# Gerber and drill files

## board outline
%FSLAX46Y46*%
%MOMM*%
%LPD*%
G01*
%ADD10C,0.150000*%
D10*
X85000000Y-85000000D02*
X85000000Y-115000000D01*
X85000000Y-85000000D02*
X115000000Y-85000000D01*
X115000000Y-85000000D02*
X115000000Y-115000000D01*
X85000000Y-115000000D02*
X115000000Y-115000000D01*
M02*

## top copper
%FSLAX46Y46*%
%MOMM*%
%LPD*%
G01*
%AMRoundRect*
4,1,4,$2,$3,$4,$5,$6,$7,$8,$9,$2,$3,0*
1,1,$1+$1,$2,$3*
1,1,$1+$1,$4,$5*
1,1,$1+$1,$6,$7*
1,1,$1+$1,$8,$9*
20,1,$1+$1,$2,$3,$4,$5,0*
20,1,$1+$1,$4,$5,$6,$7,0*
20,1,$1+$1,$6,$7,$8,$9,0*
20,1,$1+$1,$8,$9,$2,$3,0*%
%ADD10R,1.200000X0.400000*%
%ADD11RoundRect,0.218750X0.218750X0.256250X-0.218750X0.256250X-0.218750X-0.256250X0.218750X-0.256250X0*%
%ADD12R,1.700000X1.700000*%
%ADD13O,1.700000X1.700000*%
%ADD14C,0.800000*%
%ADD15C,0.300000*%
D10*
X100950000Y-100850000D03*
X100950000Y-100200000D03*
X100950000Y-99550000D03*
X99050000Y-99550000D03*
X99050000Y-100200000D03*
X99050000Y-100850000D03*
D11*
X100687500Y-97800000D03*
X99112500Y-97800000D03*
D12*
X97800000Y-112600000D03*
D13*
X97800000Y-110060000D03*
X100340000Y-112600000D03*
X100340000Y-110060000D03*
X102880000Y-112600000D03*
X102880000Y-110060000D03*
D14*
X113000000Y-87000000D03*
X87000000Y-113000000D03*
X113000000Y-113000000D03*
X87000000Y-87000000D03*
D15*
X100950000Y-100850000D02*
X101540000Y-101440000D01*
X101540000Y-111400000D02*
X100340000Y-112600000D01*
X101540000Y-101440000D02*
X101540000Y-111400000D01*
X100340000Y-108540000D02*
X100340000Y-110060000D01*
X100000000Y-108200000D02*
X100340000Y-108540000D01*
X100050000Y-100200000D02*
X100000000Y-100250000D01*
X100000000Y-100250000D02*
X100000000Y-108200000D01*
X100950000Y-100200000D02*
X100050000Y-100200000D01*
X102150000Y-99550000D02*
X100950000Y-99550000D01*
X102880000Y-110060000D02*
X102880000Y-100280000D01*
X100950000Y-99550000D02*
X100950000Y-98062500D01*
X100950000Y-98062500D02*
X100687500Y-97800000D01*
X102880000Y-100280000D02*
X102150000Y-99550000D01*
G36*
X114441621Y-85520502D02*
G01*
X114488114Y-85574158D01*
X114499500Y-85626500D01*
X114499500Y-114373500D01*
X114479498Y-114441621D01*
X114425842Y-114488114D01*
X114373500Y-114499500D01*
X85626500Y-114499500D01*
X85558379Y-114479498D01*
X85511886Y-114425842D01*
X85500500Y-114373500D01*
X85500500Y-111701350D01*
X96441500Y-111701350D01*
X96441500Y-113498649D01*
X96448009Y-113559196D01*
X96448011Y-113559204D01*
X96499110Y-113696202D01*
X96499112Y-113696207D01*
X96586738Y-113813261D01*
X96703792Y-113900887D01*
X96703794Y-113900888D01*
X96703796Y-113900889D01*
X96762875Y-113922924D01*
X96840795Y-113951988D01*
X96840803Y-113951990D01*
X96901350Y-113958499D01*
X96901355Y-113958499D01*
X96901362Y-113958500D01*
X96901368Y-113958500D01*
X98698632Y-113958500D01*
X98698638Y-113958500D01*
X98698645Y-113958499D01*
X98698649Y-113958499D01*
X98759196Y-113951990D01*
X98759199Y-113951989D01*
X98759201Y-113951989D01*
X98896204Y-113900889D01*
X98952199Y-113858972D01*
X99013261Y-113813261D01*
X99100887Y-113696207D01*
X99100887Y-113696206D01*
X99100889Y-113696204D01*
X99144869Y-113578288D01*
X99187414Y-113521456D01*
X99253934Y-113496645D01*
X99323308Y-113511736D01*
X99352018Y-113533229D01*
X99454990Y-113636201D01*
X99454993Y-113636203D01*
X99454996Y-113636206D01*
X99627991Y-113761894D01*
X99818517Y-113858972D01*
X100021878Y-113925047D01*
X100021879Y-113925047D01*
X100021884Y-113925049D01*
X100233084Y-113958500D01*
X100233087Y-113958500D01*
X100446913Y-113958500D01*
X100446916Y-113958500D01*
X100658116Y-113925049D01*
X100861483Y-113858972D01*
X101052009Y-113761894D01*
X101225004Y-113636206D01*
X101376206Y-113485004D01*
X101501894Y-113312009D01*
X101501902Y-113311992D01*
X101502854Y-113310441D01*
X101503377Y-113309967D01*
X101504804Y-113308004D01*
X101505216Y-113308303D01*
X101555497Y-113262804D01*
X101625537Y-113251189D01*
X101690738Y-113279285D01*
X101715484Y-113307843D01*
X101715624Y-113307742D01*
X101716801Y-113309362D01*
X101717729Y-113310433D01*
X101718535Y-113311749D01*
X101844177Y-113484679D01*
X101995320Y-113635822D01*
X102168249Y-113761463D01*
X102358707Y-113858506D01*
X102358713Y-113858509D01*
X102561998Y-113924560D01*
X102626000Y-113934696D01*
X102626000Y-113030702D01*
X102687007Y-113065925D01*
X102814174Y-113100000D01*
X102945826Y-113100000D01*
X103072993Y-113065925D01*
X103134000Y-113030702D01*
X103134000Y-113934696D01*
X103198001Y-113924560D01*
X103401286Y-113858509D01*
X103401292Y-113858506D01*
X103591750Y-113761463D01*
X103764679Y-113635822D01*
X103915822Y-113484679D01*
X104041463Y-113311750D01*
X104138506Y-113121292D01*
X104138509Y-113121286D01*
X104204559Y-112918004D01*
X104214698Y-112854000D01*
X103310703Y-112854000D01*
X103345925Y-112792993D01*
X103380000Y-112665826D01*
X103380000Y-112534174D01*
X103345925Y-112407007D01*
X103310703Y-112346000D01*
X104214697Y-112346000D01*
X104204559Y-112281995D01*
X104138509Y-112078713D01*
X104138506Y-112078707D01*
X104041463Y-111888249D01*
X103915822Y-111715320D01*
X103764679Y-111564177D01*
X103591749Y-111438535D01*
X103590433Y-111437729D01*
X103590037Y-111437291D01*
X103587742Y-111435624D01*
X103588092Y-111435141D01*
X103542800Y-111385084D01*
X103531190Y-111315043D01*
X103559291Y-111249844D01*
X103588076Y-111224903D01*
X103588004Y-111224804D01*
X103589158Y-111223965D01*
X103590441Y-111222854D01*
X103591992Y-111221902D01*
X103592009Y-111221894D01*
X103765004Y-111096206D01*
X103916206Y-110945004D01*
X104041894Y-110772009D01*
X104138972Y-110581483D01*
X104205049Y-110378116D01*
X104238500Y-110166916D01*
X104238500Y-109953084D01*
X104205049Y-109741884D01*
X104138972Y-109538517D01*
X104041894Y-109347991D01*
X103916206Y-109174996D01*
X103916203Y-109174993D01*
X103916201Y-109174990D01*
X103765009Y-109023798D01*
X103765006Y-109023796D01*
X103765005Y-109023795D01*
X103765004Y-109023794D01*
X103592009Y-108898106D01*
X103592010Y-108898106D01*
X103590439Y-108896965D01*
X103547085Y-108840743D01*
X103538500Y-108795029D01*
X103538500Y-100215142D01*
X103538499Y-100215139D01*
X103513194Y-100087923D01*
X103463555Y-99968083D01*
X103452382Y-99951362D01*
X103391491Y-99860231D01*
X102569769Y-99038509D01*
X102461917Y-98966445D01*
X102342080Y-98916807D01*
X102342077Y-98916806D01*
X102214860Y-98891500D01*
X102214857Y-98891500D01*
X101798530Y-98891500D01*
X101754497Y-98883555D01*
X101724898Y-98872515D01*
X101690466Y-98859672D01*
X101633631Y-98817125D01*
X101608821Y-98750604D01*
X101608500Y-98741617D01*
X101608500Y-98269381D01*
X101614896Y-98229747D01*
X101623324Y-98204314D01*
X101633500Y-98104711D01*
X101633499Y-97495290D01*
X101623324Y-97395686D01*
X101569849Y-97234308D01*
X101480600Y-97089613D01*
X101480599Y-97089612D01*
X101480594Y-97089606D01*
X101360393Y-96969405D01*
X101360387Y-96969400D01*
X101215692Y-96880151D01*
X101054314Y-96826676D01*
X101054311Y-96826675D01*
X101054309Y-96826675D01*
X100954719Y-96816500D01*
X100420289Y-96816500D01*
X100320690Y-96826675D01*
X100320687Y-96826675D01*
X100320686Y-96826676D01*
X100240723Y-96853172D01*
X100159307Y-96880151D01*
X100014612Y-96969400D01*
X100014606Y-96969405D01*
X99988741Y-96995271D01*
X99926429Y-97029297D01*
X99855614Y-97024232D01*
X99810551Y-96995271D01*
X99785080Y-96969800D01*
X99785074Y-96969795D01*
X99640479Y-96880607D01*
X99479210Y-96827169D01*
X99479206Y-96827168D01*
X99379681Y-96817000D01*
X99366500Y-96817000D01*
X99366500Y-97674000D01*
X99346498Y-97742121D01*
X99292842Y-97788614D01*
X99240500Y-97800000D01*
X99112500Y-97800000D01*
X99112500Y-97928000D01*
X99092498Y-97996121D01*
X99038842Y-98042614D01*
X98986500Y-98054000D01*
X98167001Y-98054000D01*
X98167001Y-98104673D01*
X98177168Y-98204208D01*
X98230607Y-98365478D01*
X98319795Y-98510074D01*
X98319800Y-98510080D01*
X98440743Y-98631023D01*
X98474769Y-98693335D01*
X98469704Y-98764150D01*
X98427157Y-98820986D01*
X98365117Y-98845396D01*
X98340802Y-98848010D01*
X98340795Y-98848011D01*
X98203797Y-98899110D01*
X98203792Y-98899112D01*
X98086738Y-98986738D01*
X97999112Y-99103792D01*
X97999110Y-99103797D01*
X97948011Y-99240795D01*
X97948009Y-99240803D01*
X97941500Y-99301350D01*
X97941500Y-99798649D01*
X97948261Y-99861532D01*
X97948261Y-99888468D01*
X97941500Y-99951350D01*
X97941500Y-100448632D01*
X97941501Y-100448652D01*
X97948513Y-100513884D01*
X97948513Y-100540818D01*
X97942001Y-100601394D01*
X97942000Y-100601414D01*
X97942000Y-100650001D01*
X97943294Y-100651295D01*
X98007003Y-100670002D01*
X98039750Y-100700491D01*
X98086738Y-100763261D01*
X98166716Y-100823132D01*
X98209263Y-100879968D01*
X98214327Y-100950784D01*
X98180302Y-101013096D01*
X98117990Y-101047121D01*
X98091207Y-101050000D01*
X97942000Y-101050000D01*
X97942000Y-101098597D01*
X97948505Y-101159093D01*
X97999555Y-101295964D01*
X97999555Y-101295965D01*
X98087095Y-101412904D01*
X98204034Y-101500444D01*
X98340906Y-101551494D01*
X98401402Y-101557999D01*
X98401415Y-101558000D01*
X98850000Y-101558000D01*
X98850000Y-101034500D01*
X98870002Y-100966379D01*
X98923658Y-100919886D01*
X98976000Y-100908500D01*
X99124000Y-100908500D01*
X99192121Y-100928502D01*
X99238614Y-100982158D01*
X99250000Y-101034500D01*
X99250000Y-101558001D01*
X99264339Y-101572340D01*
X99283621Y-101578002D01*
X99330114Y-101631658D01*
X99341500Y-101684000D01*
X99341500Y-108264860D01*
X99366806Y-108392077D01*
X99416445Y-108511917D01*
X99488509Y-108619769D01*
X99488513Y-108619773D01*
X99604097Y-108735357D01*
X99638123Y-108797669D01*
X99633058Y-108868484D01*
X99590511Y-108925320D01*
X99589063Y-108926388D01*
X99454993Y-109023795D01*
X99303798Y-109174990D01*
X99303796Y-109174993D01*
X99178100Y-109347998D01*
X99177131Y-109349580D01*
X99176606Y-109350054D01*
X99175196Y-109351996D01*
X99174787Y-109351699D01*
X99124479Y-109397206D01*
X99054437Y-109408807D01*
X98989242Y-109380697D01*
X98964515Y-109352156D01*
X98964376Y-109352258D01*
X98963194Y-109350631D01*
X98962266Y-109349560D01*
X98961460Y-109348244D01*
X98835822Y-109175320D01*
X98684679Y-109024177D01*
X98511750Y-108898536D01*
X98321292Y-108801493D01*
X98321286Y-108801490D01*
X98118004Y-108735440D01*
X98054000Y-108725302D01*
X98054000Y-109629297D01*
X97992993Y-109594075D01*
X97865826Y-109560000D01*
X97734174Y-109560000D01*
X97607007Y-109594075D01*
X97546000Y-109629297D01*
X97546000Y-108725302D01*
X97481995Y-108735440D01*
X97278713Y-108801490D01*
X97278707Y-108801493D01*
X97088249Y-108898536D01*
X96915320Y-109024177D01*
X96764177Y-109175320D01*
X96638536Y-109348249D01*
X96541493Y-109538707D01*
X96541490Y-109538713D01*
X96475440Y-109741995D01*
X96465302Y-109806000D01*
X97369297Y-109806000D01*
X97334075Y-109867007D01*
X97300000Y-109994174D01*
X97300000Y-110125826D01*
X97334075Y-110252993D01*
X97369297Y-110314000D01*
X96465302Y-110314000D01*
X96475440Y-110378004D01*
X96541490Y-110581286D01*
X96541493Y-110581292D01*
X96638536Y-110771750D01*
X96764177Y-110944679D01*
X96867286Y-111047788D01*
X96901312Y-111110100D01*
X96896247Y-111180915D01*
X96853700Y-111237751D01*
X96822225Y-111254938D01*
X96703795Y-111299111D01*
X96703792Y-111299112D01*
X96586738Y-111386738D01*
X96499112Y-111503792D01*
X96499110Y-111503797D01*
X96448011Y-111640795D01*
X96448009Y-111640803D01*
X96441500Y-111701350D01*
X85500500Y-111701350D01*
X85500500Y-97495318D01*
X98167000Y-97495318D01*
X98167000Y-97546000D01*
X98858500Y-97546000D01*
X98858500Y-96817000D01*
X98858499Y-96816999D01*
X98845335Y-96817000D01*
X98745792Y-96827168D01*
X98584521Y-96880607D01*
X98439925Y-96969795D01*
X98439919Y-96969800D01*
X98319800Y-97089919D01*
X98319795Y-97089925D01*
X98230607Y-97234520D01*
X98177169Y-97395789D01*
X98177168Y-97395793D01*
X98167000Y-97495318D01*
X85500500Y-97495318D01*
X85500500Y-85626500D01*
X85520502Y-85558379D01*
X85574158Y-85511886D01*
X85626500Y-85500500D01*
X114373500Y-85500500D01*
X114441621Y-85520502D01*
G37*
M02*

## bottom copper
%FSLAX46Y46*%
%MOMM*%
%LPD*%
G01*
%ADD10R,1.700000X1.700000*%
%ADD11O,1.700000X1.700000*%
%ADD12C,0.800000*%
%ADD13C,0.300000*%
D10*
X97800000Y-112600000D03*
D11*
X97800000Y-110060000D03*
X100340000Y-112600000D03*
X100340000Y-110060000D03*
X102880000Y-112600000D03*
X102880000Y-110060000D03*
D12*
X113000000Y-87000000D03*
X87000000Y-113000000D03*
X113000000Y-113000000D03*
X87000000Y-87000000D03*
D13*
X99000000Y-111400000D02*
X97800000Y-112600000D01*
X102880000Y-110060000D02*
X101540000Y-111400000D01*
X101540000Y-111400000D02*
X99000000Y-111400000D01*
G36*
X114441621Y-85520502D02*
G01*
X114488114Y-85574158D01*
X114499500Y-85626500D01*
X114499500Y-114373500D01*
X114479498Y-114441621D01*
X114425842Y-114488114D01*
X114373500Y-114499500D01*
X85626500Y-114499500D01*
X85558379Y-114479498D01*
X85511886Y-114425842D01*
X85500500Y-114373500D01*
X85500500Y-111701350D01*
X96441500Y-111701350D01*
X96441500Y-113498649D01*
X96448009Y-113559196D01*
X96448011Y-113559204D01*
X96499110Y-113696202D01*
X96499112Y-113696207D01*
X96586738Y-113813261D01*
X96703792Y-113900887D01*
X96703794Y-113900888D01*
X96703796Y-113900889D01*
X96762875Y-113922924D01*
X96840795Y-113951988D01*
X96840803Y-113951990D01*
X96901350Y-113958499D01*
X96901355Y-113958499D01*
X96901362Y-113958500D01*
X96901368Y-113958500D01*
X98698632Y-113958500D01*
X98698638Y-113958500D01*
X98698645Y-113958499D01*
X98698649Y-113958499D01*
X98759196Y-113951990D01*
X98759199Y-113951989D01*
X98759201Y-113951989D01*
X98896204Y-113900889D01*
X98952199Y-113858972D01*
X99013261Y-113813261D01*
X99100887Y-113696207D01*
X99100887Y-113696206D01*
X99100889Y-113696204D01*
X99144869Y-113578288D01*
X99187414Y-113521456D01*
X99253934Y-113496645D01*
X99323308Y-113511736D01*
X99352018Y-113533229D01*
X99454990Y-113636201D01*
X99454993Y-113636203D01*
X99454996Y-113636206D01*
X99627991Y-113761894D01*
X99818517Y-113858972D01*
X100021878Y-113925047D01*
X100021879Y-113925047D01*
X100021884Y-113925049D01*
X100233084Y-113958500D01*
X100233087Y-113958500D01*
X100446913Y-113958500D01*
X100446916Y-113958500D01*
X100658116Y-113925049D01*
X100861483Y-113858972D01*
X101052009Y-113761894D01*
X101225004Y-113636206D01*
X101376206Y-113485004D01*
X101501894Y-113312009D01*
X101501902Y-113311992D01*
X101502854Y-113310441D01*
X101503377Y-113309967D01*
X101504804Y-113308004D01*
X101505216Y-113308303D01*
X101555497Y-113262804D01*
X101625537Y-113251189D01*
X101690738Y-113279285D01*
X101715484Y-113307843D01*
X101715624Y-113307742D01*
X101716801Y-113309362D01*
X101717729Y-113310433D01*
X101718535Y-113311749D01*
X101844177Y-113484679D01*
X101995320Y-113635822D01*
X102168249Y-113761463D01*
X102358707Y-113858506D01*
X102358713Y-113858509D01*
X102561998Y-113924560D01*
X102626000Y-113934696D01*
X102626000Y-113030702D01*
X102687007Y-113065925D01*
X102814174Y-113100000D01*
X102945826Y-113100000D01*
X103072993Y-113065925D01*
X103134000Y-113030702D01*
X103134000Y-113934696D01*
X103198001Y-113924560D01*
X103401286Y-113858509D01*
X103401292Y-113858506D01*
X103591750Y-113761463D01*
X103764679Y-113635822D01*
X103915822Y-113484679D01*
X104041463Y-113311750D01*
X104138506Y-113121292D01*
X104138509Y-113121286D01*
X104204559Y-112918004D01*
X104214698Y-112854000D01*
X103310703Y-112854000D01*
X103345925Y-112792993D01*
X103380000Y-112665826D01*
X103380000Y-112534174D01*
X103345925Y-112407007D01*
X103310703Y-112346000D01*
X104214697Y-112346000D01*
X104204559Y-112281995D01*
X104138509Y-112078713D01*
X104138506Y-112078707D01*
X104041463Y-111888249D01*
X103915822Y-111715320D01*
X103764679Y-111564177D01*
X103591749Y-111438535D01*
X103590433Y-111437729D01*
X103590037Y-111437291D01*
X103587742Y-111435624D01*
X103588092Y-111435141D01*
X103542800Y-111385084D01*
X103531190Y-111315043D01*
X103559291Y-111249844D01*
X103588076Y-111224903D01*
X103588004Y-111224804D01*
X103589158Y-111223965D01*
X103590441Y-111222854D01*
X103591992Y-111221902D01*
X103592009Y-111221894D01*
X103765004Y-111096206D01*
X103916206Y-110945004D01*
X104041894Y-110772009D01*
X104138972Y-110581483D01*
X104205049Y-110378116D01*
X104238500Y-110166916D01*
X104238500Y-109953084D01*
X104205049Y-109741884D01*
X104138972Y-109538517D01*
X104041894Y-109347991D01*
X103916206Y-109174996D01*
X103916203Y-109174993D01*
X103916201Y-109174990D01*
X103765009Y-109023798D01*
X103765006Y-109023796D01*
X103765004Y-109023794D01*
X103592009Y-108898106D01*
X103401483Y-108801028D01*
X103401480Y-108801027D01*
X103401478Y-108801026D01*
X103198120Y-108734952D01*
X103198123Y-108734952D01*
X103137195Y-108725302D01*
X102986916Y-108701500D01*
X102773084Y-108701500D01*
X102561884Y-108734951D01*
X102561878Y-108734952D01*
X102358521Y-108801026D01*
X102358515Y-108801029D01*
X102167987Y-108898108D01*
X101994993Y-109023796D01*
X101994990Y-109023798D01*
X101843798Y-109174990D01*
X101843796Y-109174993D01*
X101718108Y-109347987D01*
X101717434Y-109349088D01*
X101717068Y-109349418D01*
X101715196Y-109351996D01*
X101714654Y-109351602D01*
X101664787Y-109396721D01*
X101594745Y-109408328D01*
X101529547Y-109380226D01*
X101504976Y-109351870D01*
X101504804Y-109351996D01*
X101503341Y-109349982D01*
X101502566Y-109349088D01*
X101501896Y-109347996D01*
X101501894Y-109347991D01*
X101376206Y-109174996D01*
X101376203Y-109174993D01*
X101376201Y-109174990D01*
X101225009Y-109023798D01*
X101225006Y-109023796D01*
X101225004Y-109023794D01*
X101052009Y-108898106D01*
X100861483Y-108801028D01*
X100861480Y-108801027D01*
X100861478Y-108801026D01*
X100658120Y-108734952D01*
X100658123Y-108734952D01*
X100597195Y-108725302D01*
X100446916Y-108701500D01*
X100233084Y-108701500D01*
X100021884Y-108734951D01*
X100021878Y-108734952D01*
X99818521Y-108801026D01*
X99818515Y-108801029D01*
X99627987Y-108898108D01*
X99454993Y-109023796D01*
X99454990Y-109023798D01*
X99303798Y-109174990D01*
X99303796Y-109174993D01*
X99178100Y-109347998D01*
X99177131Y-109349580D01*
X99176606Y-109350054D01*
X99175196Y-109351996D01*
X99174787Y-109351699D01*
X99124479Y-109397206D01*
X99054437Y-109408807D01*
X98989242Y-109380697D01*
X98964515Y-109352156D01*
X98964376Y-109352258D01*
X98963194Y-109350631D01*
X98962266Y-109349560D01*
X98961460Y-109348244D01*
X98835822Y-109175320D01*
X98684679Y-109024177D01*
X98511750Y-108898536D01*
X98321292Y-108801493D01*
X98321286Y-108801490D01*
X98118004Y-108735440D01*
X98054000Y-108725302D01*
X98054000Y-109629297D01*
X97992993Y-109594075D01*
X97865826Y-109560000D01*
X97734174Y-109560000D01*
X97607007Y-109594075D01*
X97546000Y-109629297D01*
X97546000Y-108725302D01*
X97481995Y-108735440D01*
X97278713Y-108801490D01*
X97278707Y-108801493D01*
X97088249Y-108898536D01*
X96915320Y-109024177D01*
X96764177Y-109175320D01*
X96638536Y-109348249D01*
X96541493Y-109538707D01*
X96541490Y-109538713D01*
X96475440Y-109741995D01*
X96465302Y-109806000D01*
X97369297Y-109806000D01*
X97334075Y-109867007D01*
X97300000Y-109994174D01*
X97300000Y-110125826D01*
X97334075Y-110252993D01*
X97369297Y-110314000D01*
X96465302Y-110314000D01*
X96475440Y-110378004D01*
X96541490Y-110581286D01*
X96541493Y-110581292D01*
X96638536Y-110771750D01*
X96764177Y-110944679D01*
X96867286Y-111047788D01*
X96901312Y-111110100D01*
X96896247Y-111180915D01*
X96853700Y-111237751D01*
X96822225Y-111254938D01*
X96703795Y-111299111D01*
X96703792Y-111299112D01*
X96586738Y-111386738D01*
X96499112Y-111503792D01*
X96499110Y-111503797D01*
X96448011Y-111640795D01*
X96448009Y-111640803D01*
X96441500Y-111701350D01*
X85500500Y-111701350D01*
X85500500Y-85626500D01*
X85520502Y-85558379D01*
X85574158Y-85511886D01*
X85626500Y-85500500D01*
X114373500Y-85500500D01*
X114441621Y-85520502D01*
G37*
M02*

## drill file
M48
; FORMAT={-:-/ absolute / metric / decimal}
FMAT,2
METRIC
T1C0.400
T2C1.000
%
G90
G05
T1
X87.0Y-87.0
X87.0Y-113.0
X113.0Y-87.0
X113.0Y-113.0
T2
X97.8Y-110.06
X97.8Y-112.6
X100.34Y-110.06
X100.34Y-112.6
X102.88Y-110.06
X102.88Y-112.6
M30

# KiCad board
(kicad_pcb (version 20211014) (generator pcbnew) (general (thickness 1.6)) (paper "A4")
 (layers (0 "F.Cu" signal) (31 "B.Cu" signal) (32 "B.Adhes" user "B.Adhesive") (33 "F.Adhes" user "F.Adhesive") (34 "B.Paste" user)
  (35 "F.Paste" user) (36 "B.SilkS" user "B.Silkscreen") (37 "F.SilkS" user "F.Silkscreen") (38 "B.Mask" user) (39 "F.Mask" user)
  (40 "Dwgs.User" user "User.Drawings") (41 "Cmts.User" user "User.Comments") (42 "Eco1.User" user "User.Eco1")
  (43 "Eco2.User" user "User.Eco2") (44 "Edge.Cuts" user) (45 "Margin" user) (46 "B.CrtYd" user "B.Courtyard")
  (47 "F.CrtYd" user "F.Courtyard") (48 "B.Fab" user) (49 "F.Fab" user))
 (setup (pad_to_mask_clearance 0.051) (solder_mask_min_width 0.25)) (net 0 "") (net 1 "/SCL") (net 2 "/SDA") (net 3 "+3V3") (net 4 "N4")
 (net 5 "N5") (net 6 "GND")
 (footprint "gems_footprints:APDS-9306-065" (layer "F.Cu") (at 100 100.2 -90)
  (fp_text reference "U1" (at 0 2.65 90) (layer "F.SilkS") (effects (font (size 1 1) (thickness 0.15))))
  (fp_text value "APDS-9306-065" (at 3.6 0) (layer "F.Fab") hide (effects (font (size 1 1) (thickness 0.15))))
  (pad "1" smd rect (at 0.65 -0.95 270) (size 0.4 1.2) (layers "F.Cu" "F.Paste" "F.Mask") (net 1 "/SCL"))
  (pad "2" smd rect (at 0 -0.95 270) (size 0.4 1.2) (layers "F.Cu" "F.Paste" "F.Mask") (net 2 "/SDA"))
  (pad "3" smd rect (at -0.65 -0.95 270) (size 0.4 1.2) (layers "F.Cu" "F.Paste" "F.Mask") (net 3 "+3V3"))
  (pad "4" smd rect (at -0.65 0.95 270) (size 0.4 1.2) (layers "F.Cu" "F.Paste" "F.Mask") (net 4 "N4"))
  (pad "5" smd rect (at 0 0.95 270) (size 0.4 1.2) (layers "F.Cu" "F.Paste" "F.Mask") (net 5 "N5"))
  (pad "6" smd rect (at 0.65 0.95 270) (size 0.4 1.2) (layers "F.Cu" "F.Paste" "F.Mask") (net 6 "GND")))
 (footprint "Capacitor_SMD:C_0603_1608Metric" (layer "F.Cu") (at 99.9 97.8 180)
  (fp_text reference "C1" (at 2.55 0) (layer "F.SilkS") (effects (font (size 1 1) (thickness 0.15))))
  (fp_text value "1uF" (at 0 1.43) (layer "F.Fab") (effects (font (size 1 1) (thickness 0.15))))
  (pad "1" smd roundrect locked (at -0.7875 0 180) (size 0.875 0.95) (layers "F.Cu" "F.Paste" "F.Mask") (roundrect_rratio 0.25)
   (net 3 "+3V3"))
  (pad "2" smd roundrect locked (at 0.7875 0 180) (size 0.875 0.95) (layers "F.Cu" "F.Paste" "F.Mask") (roundrect_rratio 0.25) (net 6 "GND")))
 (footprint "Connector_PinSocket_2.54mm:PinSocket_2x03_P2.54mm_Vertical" (layer "B.Cu") (at 97.8 112.6 -90)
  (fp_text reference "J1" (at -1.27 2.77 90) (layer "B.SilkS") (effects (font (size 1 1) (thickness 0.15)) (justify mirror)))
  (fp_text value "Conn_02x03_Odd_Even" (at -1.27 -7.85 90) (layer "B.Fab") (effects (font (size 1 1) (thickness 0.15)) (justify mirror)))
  (pad "1" thru_hole rect (at 0 0 270) (size 1.7 1.7) (drill 1) (layers *.Cu *.Mask) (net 3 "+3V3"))
  (pad "2" thru_hole oval (at -2.54 0 270) (size 1.7 1.7) (drill 1) (layers *.Cu *.Mask) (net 6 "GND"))
  (pad "3" thru_hole oval (at 0 -2.54 270) (size 1.7 1.7) (drill 1) (layers *.Cu *.Mask) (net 1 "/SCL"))
  (pad "4" thru_hole oval (at -2.54 -2.54 270) (size 1.7 1.7) (drill 1) (layers *.Cu *.Mask) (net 2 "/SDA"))
  (pad "5" thru_hole oval (at 0 -5.08 270) (size 1.7 1.7) (drill 1) (layers *.Cu *.Mask) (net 6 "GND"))
  (pad "6" thru_hole oval (at -2.54 -5.08 270) (size 1.7 1.7) (drill 1) (layers *.Cu *.Mask) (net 3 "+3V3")))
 (gr_line (start 85 85) (end 85 115) (layer "Edge.Cuts") (width 0.15))
 (gr_line (start 85 85) (end 115 85) (layer "Edge.Cuts") (width 0.15))
 (gr_line (start 115 85) (end 115 115) (layer "Edge.Cuts") (width 0.15))
 (gr_line (start 85 115) (end 115 115) (layer "Edge.Cuts") (width 0.15))
 (segment (start 100.95 100.85) (end 101.54 101.44) (width 0.3) (layer "F.Cu") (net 1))
 (segment (start 101.54 111.4) (end 100.34 112.6) (width 0.3) (layer "F.Cu") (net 1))
 (segment (start 101.54 101.44) (end 101.54 111.4) (width 0.3) (layer "F.Cu") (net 1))
 (segment (start 100.34 108.54) (end 100.34 110.06) (width 0.3) (layer "F.Cu") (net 2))
 (segment (start 100 108.2) (end 100.34 108.54) (width 0.3) (layer "F.Cu") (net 2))
 (segment (start 100.05 100.2) (end 100 100.25) (width 0.3) (layer "F.Cu") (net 2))
 (segment (start 100 100.25) (end 100 108.2) (width 0.3) (layer "F.Cu") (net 2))
 (segment (start 100.95 100.2) (end 100.05 100.2) (width 0.3) (layer "F.Cu") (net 2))
 (segment (start 102.15 99.55) (end 100.95 99.55) (width 0.3) (layer "F.Cu") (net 3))
 (segment (start 102.88 110.06) (end 102.88 100.28) (width 0.3) (layer "F.Cu") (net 3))
 (segment (start 100.95 99.55) (end 100.95 98.0625) (width 0.3) (layer "F.Cu") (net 3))
 (segment (start 100.95 98.0625) (end 100.6875 97.8) (width 0.3) (layer "F.Cu") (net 3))
 (segment (start 102.88 100.28) (end 102.15 99.55) (width 0.3) (layer "F.Cu") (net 3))
 (segment (start 99 111.4) (end 97.8 112.6) (width 0.3) (layer "B.Cu") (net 3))
 (segment (start 102.88 110.06) (end 101.54 111.4) (width 0.3) (layer "B.Cu") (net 3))
 (segment (start 101.54 111.4) (end 99 111.4) (width 0.3) (layer "B.Cu") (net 3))
 (via (at 113 87) (size 0.8) (drill 0.4) (layers "F.Cu" "B.Cu") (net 6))
 (via (at 87 113) (size 0.8) (drill 0.4) (layers "F.Cu" "B.Cu") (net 6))
 (via (at 113 113) (size 0.8) (drill 0.4) (layers "F.Cu" "B.Cu") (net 6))
 (via (at 87 87) (size 0.8) (drill 0.4) (layers "F.Cu" "B.Cu") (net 6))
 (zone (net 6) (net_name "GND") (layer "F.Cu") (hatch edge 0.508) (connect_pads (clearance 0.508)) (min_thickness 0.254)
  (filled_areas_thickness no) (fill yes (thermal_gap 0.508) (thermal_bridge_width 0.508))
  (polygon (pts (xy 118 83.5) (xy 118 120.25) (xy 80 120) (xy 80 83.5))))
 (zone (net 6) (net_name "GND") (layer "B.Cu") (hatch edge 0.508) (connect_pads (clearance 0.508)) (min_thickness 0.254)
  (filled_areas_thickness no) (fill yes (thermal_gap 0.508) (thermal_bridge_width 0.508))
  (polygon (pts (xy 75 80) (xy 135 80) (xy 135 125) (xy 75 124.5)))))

